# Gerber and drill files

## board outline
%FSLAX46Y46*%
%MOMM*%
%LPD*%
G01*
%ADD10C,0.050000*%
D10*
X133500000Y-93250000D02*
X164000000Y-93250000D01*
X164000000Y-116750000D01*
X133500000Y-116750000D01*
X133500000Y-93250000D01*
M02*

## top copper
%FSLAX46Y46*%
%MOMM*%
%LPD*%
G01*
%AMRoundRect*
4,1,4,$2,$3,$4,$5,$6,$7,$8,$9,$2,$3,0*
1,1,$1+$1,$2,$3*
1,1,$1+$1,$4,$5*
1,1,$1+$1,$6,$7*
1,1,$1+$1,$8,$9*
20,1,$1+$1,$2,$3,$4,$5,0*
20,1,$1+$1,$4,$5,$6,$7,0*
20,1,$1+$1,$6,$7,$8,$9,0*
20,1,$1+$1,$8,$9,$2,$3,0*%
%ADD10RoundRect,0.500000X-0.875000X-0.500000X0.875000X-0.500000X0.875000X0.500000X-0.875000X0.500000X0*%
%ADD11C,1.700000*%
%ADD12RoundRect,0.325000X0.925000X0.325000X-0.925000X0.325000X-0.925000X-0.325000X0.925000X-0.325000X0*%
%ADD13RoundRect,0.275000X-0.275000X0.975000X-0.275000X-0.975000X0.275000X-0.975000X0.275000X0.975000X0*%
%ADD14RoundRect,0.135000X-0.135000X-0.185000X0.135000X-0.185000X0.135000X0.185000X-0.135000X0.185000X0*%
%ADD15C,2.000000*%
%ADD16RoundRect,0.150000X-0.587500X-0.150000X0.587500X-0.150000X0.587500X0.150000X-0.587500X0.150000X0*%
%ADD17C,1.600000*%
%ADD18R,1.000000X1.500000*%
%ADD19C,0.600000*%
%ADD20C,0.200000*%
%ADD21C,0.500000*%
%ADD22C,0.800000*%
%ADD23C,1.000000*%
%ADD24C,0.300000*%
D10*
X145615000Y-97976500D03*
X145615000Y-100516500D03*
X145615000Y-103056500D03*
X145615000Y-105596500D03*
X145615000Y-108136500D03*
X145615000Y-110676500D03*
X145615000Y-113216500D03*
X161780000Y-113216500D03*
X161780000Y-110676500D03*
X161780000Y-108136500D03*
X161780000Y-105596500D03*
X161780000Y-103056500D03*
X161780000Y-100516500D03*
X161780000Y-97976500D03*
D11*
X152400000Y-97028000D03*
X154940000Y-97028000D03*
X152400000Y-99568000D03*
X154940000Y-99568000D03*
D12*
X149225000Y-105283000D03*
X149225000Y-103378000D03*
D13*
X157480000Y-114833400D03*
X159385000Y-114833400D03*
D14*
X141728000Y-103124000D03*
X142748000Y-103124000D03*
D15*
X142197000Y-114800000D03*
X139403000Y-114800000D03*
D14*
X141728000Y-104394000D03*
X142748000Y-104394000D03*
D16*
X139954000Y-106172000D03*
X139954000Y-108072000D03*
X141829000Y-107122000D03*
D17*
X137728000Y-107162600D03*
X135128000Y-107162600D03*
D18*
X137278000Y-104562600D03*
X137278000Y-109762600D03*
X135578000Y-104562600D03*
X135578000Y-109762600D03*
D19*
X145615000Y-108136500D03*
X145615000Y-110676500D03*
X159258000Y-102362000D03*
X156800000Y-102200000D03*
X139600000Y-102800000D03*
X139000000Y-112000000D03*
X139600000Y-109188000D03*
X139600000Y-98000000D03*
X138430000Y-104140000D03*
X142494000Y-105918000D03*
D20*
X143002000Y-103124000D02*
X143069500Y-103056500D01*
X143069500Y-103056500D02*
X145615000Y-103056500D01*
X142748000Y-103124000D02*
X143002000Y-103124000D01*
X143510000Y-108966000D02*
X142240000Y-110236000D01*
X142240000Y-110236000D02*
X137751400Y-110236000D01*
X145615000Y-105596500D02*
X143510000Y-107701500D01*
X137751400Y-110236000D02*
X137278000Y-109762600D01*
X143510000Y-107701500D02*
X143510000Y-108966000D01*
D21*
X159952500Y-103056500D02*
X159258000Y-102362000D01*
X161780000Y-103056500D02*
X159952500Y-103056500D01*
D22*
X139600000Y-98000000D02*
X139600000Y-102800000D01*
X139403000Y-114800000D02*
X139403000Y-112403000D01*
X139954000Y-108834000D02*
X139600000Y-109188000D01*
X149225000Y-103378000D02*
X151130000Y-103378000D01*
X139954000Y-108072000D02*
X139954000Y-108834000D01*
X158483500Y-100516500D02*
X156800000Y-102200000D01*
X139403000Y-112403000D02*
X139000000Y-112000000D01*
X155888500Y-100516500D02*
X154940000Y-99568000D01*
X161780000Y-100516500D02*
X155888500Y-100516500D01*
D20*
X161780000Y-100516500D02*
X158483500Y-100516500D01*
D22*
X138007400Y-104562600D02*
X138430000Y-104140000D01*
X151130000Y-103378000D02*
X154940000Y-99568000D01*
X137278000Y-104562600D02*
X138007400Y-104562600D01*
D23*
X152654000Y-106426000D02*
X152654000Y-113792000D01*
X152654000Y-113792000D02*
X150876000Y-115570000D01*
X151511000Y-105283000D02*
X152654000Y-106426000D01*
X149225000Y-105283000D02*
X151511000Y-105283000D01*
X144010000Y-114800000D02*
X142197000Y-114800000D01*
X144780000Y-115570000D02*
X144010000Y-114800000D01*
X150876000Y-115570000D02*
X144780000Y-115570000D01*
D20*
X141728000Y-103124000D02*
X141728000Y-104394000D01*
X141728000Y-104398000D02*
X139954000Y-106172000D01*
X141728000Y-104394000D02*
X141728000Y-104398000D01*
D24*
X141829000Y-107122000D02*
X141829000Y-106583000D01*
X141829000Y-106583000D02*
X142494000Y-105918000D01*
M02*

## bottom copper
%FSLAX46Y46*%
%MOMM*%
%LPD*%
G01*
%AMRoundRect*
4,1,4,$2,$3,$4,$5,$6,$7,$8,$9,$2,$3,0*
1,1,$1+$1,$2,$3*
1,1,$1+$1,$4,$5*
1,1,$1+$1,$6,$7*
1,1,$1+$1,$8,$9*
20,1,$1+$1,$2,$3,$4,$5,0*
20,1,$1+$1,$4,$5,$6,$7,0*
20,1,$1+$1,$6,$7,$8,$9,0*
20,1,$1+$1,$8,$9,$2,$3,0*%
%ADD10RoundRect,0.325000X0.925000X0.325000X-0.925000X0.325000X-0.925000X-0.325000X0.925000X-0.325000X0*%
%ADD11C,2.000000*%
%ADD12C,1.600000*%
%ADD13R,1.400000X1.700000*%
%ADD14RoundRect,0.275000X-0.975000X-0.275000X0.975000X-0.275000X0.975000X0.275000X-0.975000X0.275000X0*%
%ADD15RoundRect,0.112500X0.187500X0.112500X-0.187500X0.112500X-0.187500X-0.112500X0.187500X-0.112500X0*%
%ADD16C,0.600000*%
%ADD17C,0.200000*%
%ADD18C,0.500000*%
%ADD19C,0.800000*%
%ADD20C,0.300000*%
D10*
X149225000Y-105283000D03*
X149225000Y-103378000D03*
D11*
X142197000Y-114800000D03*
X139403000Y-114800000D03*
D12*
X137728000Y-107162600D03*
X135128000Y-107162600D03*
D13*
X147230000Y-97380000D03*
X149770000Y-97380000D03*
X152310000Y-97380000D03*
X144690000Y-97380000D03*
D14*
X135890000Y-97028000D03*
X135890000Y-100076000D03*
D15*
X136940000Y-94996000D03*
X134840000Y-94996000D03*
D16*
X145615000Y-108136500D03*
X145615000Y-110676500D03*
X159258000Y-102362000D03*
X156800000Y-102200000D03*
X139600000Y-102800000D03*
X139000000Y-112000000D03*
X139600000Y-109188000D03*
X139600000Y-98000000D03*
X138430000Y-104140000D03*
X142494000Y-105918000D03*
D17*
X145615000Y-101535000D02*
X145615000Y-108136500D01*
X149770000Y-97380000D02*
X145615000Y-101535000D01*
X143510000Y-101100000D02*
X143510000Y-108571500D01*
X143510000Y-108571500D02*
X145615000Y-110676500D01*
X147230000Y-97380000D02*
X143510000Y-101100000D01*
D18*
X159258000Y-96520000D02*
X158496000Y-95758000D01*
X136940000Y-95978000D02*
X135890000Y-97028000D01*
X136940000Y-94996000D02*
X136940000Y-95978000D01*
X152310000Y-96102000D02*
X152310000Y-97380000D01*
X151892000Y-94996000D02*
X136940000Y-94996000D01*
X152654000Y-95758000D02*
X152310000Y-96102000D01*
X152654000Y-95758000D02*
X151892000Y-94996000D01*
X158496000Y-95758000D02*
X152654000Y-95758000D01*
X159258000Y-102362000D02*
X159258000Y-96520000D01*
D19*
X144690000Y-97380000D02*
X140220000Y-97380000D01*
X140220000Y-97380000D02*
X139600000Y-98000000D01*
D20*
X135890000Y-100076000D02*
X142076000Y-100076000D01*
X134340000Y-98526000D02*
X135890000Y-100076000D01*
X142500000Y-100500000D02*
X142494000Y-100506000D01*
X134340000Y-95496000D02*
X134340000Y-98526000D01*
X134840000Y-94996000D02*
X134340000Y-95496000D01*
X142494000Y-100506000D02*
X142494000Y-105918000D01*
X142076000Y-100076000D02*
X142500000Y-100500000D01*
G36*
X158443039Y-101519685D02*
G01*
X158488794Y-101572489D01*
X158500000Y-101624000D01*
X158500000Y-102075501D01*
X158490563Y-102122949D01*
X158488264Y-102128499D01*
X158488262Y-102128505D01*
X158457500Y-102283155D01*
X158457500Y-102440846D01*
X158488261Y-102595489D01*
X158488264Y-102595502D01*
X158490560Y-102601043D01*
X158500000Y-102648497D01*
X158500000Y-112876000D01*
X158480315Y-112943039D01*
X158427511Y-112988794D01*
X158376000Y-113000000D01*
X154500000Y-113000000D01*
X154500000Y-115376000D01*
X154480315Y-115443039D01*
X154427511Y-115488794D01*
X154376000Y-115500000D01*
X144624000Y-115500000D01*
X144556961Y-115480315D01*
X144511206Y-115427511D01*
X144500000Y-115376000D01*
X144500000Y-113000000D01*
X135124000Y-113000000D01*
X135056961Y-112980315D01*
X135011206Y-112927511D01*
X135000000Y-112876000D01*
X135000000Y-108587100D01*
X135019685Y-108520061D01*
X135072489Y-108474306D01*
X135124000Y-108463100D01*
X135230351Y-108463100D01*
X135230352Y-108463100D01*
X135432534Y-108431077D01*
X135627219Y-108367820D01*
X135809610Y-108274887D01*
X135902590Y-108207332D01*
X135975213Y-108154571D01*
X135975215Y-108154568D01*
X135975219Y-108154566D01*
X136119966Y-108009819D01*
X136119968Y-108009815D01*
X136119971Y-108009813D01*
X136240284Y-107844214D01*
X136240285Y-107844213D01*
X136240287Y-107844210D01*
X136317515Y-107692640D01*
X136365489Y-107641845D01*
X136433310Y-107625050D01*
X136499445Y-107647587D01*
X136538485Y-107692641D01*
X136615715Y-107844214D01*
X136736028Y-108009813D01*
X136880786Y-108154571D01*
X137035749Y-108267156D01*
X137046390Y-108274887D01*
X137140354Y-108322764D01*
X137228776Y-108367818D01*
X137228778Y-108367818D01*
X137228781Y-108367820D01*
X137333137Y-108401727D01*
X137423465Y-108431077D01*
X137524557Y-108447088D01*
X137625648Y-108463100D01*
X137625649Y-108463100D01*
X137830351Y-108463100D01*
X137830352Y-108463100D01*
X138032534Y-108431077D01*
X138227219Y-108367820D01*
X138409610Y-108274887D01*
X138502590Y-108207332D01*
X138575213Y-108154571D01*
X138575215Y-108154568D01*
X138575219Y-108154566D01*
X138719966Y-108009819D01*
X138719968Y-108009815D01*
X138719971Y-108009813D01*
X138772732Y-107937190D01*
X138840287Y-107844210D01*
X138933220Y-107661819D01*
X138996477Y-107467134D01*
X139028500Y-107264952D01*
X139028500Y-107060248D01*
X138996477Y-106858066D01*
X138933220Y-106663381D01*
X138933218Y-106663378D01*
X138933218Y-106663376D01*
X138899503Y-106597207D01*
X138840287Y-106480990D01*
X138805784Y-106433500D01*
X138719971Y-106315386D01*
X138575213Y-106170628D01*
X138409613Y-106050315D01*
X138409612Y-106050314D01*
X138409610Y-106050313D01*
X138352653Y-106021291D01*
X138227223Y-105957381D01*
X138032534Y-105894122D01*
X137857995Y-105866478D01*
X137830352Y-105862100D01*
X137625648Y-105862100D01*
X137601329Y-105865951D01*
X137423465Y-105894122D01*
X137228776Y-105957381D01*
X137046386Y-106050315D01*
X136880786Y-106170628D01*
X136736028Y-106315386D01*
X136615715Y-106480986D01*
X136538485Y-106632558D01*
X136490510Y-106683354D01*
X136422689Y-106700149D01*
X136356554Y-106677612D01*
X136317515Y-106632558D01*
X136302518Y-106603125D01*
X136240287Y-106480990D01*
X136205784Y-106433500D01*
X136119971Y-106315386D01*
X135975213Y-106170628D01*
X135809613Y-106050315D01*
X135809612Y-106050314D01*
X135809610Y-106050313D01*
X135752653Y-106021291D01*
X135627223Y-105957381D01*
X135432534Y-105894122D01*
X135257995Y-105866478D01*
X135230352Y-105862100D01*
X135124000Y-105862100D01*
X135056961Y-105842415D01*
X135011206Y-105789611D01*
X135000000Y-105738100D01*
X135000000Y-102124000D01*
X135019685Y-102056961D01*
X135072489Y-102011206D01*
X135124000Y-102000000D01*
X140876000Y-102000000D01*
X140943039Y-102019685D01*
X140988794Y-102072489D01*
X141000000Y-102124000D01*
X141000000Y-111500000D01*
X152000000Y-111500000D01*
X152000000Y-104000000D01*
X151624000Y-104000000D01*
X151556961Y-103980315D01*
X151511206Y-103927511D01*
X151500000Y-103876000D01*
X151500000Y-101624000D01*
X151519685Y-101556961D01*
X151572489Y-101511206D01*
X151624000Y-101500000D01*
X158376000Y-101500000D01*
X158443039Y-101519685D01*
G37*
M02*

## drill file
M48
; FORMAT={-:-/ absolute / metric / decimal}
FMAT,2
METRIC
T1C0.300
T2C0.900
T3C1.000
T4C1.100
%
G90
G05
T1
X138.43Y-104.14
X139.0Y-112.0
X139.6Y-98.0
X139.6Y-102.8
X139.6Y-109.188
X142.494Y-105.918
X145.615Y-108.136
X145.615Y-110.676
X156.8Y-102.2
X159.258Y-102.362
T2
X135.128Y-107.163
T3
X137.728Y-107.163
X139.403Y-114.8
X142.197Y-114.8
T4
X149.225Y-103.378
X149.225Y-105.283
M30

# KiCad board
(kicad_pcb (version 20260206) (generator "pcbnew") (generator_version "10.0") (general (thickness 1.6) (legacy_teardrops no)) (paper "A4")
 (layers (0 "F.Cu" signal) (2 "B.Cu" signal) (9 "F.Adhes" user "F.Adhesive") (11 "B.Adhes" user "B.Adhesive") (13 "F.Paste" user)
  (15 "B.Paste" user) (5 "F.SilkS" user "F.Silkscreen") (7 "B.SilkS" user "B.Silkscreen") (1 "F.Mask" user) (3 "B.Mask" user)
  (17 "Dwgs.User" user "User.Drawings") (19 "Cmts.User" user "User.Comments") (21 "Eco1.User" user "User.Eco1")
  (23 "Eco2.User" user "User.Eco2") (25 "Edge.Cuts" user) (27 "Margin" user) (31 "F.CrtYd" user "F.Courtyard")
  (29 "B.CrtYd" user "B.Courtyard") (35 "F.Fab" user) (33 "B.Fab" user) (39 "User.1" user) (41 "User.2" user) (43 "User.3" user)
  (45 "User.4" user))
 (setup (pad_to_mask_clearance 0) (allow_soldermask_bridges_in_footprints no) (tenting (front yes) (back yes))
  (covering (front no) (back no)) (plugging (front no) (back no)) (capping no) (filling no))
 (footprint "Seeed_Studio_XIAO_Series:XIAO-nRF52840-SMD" (layer "F.Cu") (at 144.78 116.0965)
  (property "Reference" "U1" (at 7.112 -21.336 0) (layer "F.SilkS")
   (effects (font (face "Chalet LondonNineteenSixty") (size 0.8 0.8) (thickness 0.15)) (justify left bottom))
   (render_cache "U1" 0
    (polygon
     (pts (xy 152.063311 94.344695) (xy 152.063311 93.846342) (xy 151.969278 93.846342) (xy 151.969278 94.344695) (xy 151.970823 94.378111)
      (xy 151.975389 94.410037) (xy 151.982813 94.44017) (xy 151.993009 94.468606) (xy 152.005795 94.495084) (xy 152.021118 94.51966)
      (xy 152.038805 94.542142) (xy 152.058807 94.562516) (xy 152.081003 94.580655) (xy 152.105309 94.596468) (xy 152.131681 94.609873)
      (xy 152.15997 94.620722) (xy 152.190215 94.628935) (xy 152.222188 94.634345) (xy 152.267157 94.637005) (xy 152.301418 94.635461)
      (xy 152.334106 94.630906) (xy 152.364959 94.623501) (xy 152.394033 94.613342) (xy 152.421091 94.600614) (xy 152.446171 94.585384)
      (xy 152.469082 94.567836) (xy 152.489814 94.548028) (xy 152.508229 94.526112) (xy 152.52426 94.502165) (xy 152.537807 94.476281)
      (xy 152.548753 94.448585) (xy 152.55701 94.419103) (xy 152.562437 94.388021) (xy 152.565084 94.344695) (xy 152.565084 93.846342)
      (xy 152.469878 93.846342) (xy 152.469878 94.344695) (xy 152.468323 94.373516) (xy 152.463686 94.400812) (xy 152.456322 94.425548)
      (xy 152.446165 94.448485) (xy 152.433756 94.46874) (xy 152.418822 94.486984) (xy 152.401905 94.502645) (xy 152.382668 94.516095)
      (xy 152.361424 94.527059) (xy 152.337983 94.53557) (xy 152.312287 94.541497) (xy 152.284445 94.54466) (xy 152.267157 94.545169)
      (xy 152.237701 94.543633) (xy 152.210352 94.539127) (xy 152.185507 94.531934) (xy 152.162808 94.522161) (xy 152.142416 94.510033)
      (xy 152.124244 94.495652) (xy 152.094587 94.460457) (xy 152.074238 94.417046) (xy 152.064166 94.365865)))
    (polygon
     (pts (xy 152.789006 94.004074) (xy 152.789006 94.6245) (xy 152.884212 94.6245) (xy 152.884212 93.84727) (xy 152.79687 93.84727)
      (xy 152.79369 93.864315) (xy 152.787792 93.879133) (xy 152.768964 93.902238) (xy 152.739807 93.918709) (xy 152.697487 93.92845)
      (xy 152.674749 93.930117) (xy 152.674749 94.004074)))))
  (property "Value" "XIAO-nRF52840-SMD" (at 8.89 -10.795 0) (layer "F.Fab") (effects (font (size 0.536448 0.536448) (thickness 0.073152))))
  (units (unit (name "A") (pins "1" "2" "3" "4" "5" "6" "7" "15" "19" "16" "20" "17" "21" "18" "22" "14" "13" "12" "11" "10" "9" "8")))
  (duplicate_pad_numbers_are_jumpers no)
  (pad "1" smd roundrect (at 0.835 -18.12) (size 2.75 2) (layers "F.Cu" "F.Mask" "F.Paste") (roundrect_rratio 0.25)
   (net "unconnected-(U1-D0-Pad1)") (solder_mask_margin 0.0508) (thermal_bridge_angle 45))
  (pad "2" smd roundrect (at 0.835 -15.58) (size 2.75 2) (layers "F.Cu" "F.Mask" "F.Paste") (roundrect_rratio 0.25)
   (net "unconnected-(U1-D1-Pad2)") (solder_mask_margin 0.0508) (thermal_bridge_angle 45))
  (pad "3" smd roundrect (at 0.835 -13.04) (size 2.75 2) (layers "F.Cu" "F.Mask" "F.Paste") (roundrect_rratio 0.25) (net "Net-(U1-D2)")
   (solder_mask_margin 0.0508) (thermal_bridge_angle 45))
  (pad "4" smd roundrect (at 0.835 -10.5) (size 2.75 2) (layers "F.Cu" "F.Mask" "F.Paste") (roundrect_rratio 0.25) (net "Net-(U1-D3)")
   (solder_mask_margin 0.0508) (thermal_bridge_angle 45))
  (pad "5" smd roundrect (at 0.835 -7.96) (size 2.75 2) (layers "F.Cu" "F.Mask" "F.Paste") (roundrect_rratio 0.25) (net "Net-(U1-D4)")
   (solder_mask_margin 0.0508) (thermal_bridge_angle 45))
  (pad "6" smd roundrect (at 0.835 -5.42) (size 2.75 2) (layers "F.Cu" "F.Mask" "F.Paste") (roundrect_rratio 0.25) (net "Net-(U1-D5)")
   (solder_mask_margin 0.0508) (thermal_bridge_angle 45))
  (pad "7" smd roundrect (at 0.835 -2.88) (size 2.75 2) (layers "F.Cu" "F.Mask" "F.Paste") (roundrect_rratio 0.25)
   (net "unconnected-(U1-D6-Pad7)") (solder_mask_margin 0.0508) (thermal_bridge_angle 45))
  (pad "8" smd roundrect (at 17 -2.88) (size 2.75 2) (layers "F.Cu" "F.Mask" "F.Paste") (roundrect_rratio 0.25)
   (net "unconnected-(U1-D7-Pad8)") (solder_mask_margin 0.0508) (thermal_bridge_angle 45))
  (pad "9" smd roundrect (at 17 -5.42) (size 2.75 2) (layers "F.Cu" "F.Mask" "F.Paste") (roundrect_rratio 0.25)
   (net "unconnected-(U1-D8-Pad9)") (solder_mask_margin 0.0508) (thermal_bridge_angle 45))
  (pad "10" smd roundrect (at 17 -7.96) (size 2.75 2) (layers "F.Cu" "F.Mask" "F.Paste") (roundrect_rratio 0.25)
   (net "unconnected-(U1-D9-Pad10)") (solder_mask_margin 0.0508) (thermal_bridge_angle 45))
  (pad "11" smd roundrect (at 17 -10.5) (size 2.75 2) (layers "F.Cu" "F.Mask" "F.Paste") (roundrect_rratio 0.25)
   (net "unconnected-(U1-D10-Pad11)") (solder_mask_margin 0.0508) (thermal_bridge_angle 45))
  (pad "12" smd roundrect (at 17 -13.04) (size 2.75 2) (layers "F.Cu" "F.Mask" "F.Paste") (roundrect_rratio 0.25) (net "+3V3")
   (solder_mask_margin 0.0508) (thermal_bridge_angle 45))
  (pad "13" smd roundrect (at 17 -15.58) (size 2.75 2) (layers "F.Cu" "F.Mask" "F.Paste") (roundrect_rratio 0.25) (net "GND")
   (solder_mask_margin 0.0508) (thermal_bridge_angle 45))
  (pad "14" smd roundrect (at 17 -18.12) (size 2.75 2) (layers "F.Cu" "F.Mask" "F.Paste") (roundrect_rratio 0.25)
   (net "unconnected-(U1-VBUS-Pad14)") (solder_mask_margin 0.0508) (thermal_bridge_angle 45))
  (pad "15" smd circle (at 7.62 -19.0685) (size 1.7 1.7) (layers "F.Cu" "F.Mask" "F.Paste") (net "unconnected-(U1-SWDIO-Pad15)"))
  (pad "16" smd circle (at 10.16 -19.0685) (size 1.7 1.7) (layers "F.Cu" "F.Mask" "F.Paste") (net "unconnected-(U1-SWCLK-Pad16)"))
  (pad "17" smd circle (at 7.62 -16.5285) (size 1.7 1.7) (layers "F.Cu" "F.Mask" "F.Paste") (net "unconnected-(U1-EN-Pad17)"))
  (pad "18" smd circle (at 10.16 -16.5285) (size 1.7 1.7) (layers "F.Cu" "F.Mask" "F.Paste") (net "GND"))
  (pad "19" thru_hole roundrect (at 4.445 -10.8135 180) (size 2.5 1.3) (drill 1.1) (layers "*.Cu" "F.Mask" "F.Paste")
   (remove_unused_layers no) (roundrect_rratio 0.25) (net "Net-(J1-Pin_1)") (thermal_bridge_angle 45))
  (pad "20" thru_hole roundrect (at 4.445 -12.7185 180) (size 2.5 1.3) (drill 1.1) (layers "*.Cu" "F.Mask" "F.Paste")
   (remove_unused_layers no) (roundrect_rratio 0.25) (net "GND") (thermal_bridge_angle 45))
  (pad "21" smd roundrect (at 12.7 -1.2631 270) (size 2.5 1.1) (layers "F.Cu" "F.Mask" "F.Paste") (roundrect_rratio 0.25)
   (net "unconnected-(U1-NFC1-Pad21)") (thermal_bridge_angle 45))
  (pad "22" smd roundrect (at 14.605 -1.2631 270) (size 2.5 1.1) (layers "F.Cu" "F.Mask" "F.Paste") (roundrect_rratio 0.25)
   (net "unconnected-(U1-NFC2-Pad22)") (thermal_bridge_angle 45)))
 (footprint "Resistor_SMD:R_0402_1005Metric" (layer "F.Cu") (at 142.238 103.124)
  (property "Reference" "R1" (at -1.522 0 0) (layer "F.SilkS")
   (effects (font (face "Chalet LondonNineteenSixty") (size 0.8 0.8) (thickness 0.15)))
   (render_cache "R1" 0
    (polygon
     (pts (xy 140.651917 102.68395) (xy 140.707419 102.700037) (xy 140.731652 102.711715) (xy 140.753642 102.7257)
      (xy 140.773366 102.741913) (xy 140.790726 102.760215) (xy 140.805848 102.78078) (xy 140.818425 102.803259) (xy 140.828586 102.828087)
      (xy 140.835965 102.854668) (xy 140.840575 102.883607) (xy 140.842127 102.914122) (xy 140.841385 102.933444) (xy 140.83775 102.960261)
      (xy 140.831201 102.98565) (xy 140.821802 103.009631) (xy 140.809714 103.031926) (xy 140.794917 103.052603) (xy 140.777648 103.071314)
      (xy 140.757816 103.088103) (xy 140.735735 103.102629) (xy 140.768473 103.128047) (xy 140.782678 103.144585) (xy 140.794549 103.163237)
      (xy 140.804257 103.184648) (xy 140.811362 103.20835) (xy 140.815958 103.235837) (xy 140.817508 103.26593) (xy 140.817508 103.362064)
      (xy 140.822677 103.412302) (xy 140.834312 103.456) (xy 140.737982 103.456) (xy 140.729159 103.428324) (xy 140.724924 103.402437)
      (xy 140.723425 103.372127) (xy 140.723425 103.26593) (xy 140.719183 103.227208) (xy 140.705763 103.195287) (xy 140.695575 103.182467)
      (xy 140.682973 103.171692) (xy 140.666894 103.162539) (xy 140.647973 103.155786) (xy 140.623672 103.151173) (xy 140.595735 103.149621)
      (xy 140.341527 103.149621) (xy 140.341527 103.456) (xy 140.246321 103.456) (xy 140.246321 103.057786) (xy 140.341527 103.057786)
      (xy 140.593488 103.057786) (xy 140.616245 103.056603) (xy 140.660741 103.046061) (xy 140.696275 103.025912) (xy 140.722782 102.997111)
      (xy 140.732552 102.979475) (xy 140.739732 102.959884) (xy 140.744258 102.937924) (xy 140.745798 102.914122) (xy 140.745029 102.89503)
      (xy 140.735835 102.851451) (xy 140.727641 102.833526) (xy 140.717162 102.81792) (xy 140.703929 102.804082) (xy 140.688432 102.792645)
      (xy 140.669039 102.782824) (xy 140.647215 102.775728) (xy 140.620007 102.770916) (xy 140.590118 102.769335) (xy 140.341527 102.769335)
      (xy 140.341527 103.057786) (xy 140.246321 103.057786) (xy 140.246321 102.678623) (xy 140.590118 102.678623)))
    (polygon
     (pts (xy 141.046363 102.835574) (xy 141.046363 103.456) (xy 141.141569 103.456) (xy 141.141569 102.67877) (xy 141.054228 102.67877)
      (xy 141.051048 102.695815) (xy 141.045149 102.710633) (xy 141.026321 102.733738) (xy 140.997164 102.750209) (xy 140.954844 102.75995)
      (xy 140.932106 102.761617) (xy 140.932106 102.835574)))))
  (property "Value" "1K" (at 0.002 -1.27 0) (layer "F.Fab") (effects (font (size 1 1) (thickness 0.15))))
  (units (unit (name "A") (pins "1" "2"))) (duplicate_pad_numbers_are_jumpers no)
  (pad "1" smd roundrect (at -0.51 0) (size 0.54 0.64) (layers "F.Cu" "F.Mask" "F.Paste") (roundrect_rratio 0.25) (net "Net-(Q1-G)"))
  (pad "2" smd roundrect (at 0.51 0) (size 0.54 0.64) (layers "F.Cu" "F.Mask" "F.Paste") (roundrect_rratio 0.25) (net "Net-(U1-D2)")))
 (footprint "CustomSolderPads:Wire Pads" (layer "F.Cu") (at 140.8 114.8 -90)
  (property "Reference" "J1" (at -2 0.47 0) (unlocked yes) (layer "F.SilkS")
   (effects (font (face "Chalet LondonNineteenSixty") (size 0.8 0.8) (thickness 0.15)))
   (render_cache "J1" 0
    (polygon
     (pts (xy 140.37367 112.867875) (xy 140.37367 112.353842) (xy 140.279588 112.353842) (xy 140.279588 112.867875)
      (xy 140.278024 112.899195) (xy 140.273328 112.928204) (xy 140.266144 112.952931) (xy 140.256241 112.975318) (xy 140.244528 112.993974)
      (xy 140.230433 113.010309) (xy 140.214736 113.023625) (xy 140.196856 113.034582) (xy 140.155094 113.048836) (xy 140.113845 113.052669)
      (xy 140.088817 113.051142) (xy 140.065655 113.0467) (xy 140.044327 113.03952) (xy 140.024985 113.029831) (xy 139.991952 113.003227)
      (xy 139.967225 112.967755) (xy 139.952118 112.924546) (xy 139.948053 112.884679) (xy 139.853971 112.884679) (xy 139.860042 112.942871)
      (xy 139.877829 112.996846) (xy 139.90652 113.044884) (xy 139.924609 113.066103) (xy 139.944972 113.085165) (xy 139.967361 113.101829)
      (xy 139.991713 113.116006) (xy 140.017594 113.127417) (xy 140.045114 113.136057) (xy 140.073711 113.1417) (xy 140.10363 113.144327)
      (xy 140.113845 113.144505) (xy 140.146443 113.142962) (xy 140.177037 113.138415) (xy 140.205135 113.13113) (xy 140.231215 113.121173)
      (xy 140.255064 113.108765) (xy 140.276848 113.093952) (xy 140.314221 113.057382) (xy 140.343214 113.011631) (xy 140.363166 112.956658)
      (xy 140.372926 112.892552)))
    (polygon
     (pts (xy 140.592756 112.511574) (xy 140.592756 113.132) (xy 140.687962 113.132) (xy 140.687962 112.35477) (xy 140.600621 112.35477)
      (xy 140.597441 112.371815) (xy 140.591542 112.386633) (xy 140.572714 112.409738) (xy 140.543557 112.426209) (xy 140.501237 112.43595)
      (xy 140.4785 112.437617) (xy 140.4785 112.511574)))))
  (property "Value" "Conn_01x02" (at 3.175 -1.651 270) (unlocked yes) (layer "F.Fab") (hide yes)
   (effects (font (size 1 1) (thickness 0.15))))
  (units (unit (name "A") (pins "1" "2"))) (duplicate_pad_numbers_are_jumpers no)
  (pad "1" thru_hole circle (at 0 -1.397 90) (size 2 2) (drill 1) (layers "*.Cu" "*.Mask") (remove_unused_layers no) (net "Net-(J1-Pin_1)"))
  (pad "2" thru_hole circle (at 0 1.397 90) (size 2 2) (drill 1) (layers "*.Cu" "*.Mask") (remove_unused_layers no) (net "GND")))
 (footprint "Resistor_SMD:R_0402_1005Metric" (layer "F.Cu") (at 142.238 104.394)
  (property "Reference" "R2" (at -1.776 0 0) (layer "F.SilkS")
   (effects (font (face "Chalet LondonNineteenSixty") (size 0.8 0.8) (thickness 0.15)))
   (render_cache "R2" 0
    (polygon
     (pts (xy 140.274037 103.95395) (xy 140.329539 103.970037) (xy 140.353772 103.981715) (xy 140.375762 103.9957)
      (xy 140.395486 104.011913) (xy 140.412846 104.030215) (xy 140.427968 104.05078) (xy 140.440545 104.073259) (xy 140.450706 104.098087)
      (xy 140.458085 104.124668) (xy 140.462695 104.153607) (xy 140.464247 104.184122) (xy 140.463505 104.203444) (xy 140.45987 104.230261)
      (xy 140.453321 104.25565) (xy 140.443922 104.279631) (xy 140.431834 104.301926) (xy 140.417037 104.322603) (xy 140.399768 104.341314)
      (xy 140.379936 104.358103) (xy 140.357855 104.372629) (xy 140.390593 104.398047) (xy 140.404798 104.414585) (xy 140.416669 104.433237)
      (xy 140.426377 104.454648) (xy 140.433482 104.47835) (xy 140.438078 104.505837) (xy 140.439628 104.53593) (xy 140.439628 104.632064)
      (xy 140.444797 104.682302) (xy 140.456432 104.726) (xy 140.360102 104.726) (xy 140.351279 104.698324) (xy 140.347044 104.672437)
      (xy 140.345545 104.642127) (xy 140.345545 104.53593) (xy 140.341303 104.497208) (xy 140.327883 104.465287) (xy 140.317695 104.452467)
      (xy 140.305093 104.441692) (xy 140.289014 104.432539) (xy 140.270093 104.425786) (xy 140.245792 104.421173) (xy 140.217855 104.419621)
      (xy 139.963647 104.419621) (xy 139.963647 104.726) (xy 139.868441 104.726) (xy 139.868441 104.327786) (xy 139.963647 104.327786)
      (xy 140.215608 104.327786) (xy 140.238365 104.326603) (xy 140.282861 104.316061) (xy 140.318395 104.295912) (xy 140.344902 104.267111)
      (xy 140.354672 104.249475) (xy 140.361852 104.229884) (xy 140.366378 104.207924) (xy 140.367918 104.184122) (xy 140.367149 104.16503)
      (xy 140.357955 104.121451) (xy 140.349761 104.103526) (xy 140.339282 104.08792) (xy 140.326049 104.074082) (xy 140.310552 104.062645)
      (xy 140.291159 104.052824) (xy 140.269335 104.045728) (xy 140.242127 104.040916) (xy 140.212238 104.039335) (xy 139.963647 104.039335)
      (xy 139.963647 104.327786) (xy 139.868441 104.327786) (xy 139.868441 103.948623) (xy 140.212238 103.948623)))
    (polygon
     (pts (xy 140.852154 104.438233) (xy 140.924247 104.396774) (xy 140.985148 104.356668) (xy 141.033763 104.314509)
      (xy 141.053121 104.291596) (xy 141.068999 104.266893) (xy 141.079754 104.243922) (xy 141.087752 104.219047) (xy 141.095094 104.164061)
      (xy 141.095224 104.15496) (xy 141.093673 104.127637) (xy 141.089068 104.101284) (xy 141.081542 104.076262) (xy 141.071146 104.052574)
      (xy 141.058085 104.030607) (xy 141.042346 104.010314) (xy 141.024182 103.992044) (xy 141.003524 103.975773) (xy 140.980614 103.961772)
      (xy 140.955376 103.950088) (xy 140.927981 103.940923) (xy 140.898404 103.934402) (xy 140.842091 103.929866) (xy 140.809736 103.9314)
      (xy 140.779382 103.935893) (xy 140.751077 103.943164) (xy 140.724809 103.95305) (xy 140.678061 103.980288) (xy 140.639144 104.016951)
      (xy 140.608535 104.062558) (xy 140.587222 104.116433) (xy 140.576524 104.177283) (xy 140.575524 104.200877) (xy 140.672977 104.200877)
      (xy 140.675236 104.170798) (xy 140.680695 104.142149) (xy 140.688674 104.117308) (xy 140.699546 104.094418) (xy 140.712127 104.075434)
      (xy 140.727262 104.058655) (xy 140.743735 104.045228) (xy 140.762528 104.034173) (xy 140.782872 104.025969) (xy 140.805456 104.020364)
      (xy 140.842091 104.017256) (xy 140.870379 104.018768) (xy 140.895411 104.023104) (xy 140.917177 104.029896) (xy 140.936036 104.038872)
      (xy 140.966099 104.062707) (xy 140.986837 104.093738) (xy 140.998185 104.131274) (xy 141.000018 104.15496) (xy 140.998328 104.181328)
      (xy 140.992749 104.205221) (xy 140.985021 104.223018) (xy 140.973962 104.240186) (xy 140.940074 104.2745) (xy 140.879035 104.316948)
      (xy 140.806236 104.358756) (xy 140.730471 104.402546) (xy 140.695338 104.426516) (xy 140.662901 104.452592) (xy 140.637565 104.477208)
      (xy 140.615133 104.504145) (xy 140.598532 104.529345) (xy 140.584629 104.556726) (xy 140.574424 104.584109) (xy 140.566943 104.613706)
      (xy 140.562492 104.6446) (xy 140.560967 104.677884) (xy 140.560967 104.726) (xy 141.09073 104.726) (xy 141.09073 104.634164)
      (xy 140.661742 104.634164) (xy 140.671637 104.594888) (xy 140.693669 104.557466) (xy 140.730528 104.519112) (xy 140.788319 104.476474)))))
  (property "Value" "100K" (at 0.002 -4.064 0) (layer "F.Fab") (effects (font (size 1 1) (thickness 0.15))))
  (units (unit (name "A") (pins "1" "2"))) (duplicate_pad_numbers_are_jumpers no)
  (pad "1" smd roundrect (at -0.51 0) (size 0.54 0.64) (layers "F.Cu" "F.Mask" "F.Paste") (roundrect_rratio 0.25) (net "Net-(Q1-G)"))
  (pad "2" smd roundrect (at 0.51 0) (size 0.54 0.64) (layers "F.Cu" "F.Mask" "F.Paste") (roundrect_rratio 0.25) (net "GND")))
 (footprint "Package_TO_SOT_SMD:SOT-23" (layer "F.Cu") (at 140.8915 107.122)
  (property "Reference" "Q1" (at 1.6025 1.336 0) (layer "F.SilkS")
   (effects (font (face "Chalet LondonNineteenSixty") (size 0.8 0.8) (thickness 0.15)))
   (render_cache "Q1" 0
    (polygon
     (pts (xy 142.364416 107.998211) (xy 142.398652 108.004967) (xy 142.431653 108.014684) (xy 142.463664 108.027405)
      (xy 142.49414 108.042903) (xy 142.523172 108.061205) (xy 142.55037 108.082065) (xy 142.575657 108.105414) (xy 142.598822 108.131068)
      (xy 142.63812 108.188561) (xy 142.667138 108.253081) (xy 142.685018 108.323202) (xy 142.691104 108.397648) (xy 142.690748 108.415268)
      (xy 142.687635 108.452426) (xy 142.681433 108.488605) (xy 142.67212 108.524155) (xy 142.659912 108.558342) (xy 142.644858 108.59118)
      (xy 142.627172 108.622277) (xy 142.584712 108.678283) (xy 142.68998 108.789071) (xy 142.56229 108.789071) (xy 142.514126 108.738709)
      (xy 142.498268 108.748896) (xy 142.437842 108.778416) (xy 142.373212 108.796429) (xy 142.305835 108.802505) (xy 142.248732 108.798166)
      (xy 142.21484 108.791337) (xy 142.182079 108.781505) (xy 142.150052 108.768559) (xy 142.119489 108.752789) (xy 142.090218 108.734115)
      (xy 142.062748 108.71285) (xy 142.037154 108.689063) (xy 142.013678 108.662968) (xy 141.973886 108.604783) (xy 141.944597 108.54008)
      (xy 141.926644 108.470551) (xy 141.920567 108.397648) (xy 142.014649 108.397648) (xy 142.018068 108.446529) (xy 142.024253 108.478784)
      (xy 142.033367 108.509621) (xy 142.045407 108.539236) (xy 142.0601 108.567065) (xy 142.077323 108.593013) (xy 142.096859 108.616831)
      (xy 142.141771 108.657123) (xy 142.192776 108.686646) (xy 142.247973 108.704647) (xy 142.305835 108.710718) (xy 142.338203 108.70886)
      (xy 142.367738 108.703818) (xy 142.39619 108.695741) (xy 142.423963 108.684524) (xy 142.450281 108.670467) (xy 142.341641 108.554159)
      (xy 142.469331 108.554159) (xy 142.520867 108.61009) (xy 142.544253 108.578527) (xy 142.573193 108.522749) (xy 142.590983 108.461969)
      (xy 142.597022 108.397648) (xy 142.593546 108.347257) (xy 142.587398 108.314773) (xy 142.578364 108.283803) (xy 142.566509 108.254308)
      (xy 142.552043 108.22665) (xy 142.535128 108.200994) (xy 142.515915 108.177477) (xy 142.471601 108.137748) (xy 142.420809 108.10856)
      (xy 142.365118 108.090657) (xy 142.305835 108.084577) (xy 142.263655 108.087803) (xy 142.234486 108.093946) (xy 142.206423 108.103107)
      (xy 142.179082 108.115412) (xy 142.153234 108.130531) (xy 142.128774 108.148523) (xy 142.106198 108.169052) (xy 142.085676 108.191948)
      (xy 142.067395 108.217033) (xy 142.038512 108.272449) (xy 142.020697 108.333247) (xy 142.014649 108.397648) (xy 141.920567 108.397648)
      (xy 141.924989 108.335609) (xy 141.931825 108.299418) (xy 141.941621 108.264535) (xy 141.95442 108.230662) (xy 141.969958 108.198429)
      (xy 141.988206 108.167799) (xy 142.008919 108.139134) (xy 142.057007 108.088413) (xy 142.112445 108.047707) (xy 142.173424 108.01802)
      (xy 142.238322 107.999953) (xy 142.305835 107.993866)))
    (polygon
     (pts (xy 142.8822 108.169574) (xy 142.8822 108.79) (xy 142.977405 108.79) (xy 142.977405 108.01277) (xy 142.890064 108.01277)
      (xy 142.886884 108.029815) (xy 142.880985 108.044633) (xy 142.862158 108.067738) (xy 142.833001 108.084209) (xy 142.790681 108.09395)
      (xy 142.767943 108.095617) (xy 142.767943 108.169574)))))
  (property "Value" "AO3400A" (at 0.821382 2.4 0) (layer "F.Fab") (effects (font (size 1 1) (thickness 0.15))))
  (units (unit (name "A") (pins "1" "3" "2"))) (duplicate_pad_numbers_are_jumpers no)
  (pad "1" smd roundrect (at -0.9375 -0.95) (size 1.475 0.6) (layers "F.Cu" "F.Mask" "F.Paste") (roundrect_rratio 0.25) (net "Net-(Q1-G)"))
  (pad "2" smd roundrect (at -0.9375 0.95) (size 1.475 0.6) (layers "F.Cu" "F.Mask" "F.Paste") (roundrect_rratio 0.25) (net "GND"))
  (pad "3" smd roundrect (at 0.9375 0) (size 1.475 0.6) (layers "F.Cu" "F.Mask" "F.Paste") (roundrect_rratio 0.25) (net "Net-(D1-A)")))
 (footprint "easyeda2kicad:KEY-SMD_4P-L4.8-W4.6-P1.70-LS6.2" (layer "F.Cu") (at 136.428 107.1626 -90)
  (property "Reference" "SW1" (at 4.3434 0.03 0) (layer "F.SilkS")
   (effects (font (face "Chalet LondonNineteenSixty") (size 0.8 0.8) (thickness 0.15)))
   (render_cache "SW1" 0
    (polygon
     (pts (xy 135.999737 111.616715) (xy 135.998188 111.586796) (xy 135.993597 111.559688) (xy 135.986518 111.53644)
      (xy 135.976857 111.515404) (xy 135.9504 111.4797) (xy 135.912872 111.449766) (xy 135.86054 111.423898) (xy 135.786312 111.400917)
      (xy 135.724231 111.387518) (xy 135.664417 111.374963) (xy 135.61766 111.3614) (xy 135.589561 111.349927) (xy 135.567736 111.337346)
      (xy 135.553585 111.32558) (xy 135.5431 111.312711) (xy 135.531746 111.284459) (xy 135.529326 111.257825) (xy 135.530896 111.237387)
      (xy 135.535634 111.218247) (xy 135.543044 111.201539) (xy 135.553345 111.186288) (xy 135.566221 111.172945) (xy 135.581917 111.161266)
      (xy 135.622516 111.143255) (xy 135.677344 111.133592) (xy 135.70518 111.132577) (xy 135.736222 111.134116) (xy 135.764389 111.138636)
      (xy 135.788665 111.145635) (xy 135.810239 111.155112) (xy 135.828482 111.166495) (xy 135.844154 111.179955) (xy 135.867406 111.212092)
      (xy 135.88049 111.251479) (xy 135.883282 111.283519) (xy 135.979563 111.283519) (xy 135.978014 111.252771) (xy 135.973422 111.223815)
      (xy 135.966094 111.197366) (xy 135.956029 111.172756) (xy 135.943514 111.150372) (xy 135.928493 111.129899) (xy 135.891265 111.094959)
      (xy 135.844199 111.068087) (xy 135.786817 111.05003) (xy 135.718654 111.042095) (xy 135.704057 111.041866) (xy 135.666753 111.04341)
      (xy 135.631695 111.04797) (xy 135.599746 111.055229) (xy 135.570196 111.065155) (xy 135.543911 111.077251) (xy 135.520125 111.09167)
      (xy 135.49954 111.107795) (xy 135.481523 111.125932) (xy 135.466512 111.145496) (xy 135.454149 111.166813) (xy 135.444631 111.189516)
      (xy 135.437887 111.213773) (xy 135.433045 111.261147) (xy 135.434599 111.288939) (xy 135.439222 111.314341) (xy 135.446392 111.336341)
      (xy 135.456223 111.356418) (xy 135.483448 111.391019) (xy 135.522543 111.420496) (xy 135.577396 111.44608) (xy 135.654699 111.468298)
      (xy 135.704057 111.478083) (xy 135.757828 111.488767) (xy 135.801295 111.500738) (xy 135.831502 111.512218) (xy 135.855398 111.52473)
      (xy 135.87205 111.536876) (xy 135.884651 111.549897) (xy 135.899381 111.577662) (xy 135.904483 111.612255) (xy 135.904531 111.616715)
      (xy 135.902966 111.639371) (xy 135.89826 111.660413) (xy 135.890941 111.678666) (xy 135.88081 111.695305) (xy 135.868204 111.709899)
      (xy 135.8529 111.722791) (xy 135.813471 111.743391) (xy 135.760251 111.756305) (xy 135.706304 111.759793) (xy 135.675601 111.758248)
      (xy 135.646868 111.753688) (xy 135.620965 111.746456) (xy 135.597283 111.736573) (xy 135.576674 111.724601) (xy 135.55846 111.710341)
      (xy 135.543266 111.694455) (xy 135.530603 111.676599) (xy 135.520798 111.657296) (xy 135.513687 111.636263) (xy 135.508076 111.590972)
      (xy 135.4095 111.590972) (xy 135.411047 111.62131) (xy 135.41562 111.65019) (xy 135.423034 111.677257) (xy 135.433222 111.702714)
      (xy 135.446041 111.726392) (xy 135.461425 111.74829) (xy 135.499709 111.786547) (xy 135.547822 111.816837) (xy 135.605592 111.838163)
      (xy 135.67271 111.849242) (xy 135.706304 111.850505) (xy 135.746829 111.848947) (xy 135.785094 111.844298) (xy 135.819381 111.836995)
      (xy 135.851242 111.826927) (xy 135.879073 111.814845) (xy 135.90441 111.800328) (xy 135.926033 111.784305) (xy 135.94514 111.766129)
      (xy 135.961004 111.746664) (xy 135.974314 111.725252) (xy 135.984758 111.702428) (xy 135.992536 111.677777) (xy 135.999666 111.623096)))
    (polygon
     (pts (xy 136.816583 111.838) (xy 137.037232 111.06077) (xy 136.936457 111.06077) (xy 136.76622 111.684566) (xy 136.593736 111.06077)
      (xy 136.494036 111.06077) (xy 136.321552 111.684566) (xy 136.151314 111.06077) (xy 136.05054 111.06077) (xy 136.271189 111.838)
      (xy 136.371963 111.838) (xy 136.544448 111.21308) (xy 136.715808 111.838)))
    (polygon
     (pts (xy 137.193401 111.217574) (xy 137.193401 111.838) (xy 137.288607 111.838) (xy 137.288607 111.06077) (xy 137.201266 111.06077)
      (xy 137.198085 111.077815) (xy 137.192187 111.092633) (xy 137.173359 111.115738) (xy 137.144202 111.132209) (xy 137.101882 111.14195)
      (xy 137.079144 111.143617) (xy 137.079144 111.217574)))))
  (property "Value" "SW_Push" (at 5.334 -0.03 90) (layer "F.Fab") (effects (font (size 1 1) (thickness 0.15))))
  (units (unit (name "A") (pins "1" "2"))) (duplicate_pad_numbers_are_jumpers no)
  (pad "" thru_hole circle (at 0 -1.3 270) (size 1.6 1.6) (drill 1) (layers "*.Cu" "*.Mask") (remove_unused_layers no))
  (pad "" thru_hole circle (at 0 1.3 270) (size 1.6 1.6) (drill 0.9) (layers "*.Cu" "*.Mask") (remove_unused_layers no))
  (pad "1" smd rect (at -2.6 -0.85 270) (size 1.5 1) (layers "F.Cu" "F.Mask" "F.Paste") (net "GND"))
  (pad "2" smd rect (at 2.6 -0.85 270) (size 1.5 1) (layers "F.Cu" "F.Mask" "F.Paste") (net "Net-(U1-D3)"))
  (pad "3" smd rect (at -2.6 0.85 270) (size 1.5 1) (layers "F.Cu" "F.Mask" "F.Paste"))
  (pad "4" smd rect (at 2.6 0.85 270) (size 1.5 1) (layers "F.Cu" "F.Mask" "F.Paste")))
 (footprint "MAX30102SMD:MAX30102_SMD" (layer "B.Cu") (at 148.5 105 180)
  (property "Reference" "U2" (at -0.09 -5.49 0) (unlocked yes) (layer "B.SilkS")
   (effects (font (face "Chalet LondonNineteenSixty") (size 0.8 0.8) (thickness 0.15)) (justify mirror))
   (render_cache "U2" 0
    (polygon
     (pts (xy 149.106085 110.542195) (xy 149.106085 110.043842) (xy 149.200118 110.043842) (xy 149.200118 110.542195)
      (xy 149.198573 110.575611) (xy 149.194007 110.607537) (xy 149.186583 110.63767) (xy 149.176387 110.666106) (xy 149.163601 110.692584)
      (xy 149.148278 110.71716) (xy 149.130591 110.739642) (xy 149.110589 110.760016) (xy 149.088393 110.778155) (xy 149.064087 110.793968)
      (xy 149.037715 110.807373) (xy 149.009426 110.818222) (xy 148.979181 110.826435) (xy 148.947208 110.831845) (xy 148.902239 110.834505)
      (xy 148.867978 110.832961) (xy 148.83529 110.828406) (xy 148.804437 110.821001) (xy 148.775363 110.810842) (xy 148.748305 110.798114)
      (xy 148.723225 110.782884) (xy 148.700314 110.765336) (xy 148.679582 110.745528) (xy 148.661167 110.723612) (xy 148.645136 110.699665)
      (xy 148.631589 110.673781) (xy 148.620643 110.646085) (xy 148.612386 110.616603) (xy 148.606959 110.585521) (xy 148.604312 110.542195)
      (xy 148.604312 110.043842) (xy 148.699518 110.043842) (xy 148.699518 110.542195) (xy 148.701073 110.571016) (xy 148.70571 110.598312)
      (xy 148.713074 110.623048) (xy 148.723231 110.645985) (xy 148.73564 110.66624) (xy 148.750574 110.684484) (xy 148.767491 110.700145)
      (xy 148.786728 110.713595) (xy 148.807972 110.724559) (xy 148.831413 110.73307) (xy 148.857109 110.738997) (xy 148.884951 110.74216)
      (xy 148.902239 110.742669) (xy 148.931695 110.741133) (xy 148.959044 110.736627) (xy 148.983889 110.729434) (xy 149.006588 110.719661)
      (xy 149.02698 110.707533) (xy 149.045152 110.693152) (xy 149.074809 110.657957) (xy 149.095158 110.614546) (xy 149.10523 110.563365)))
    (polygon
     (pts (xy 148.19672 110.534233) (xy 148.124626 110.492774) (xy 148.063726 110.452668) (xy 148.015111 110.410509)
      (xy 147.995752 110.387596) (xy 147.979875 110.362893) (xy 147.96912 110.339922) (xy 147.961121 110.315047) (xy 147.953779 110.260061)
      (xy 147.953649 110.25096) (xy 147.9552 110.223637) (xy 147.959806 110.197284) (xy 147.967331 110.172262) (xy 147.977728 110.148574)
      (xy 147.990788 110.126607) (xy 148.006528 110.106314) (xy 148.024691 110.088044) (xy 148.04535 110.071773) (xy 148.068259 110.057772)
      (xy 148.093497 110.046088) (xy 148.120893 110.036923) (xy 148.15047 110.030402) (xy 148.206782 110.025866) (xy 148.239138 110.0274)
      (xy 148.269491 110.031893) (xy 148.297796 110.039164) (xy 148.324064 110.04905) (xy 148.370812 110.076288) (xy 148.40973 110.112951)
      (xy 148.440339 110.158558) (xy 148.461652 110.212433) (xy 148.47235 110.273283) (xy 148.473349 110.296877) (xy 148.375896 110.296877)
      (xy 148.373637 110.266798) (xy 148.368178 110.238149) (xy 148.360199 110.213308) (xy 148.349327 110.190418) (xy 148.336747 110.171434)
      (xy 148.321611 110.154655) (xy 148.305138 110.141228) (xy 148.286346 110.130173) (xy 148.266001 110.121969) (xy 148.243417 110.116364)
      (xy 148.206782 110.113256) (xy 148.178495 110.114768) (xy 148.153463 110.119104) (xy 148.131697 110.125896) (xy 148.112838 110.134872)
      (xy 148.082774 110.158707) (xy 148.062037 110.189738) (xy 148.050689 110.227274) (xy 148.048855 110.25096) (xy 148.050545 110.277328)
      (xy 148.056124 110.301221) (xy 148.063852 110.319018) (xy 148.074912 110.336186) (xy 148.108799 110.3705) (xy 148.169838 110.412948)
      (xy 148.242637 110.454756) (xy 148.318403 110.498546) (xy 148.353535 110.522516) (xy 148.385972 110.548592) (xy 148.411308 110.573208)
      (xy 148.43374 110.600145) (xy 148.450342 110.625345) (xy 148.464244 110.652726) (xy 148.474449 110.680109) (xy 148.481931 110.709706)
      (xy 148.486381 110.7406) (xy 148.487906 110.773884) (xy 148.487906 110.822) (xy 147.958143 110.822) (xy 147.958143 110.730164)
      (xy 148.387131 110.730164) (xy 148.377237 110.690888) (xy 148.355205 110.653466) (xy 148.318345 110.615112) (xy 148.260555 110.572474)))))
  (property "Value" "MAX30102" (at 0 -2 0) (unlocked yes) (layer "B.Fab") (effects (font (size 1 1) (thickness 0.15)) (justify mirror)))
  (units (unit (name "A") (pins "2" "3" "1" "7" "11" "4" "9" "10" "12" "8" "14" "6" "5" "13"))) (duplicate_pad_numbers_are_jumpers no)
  (pad "2" smd rect (at 1.27 7.62 180) (size 1.4 1.7) (layers "B.Cu" "B.Mask") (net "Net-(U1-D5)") (thermal_bridge_angle 45))
  (pad "3" smd rect (at -1.27 7.62 180) (size 1.4 1.7) (layers "B.Cu" "B.Mask") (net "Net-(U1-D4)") (thermal_bridge_angle 45))
  (pad "11" smd rect (at -3.81 7.62 180) (size 1.4 1.7) (layers "B.Cu" "B.Mask") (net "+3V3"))
  (pad "12" smd rect (at 3.81 7.62 180) (size 1.4 1.7) (layers "B.Cu" "B.Mask") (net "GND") (thermal_bridge_angle 45))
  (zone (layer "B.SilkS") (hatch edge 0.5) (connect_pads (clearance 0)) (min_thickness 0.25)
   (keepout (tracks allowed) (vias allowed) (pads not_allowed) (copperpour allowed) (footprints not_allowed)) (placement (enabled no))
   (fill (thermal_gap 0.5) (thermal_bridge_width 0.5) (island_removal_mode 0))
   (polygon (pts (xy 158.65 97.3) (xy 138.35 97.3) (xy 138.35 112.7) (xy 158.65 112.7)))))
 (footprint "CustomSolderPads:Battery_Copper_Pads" (layer "B.Cu") (at 135.89 98.552 180)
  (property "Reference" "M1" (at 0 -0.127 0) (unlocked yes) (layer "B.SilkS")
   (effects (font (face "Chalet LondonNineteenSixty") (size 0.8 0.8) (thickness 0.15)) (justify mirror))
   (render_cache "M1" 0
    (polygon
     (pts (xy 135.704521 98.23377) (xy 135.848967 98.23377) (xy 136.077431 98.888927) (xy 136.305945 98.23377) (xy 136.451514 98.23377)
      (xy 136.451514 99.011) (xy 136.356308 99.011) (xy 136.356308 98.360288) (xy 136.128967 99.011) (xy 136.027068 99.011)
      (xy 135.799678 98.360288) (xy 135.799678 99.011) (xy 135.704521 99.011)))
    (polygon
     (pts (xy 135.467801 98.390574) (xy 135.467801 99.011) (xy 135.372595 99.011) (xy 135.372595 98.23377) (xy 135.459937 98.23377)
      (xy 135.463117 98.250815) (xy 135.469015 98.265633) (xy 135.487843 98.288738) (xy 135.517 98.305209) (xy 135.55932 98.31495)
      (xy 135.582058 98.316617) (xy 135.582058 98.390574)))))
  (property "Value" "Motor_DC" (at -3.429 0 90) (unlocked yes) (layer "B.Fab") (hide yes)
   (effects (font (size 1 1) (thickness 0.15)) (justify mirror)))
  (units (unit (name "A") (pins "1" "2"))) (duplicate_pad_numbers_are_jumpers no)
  (pad "1" smd roundrect (at 0 1.524) (size 2.5 1.1) (layers "B.Cu" "B.Mask" "B.Paste") (roundrect_rratio 0.25) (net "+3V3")
   (thermal_bridge_angle 45))
  (pad "2" smd roundrect (at 0 -1.524) (size 2.5 1.1) (layers "B.Cu" "B.Mask" "B.Paste") (roundrect_rratio 0.25) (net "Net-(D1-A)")
   (thermal_bridge_angle 45)))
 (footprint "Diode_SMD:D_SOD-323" (layer "B.Cu") (at 135.89 94.996 180)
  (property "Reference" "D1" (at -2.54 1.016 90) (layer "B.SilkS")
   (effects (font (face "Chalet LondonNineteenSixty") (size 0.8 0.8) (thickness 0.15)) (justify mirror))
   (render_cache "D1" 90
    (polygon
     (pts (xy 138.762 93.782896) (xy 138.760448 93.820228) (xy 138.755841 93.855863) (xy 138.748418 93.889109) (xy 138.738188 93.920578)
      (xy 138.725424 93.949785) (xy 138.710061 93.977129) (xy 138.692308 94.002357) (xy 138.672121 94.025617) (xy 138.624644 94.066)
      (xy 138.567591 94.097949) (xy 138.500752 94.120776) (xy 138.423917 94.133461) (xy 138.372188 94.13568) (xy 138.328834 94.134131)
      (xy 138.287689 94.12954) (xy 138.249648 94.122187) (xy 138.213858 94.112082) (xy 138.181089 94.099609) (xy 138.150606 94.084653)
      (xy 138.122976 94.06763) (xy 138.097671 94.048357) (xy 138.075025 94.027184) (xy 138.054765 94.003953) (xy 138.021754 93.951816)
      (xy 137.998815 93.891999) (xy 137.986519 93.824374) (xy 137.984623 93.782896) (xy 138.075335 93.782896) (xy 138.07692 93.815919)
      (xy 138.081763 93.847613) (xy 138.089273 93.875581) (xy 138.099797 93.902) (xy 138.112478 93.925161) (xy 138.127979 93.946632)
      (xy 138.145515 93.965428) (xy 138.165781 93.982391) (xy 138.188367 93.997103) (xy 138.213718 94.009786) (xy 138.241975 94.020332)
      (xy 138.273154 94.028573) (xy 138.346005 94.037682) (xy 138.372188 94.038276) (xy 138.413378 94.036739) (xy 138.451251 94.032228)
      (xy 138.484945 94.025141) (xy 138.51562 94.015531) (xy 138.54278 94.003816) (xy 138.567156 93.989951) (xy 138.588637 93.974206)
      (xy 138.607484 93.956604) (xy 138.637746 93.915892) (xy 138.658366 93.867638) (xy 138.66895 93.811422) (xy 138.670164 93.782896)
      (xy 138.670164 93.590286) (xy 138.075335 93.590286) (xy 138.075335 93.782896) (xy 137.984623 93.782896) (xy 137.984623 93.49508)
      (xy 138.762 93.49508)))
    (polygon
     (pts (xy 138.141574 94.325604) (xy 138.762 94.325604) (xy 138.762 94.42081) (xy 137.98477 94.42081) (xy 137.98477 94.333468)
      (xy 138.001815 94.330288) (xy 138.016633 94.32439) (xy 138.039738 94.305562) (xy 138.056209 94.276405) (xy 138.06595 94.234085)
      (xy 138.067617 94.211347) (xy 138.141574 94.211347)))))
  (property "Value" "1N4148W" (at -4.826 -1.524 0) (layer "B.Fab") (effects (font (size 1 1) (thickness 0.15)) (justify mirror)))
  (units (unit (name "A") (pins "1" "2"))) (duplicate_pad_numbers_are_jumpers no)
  (pad "1" smd roundrect (at -1.05 0 180) (size 0.6 0.45) (layers "B.Cu" "B.Mask" "B.Paste") (roundrect_rratio 0.25) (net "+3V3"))
  (pad "2" smd roundrect (at 1.05 0 180) (size 0.6 0.45) (layers "B.Cu" "B.Mask" "B.Paste") (roundrect_rratio 0.25) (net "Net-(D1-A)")))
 (gr_rect (start 133.5 93.25) (end 164 116.75) (stroke (width 0.05) (type default)) (fill no) (layer "Edge.Cuts"))
 (segment (start 143.002 103.124) (end 143.0695 103.0565) (width 0.2) (layer "F.Cu") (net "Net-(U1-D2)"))
 (segment (start 143.0695 103.0565) (end 145.615 103.0565) (width 0.2) (layer "F.Cu") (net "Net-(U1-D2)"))
 (segment (start 142.748 103.124) (end 143.002 103.124) (width 0.2) (layer "F.Cu") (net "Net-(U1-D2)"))
 (segment (start 143.51 108.966) (end 142.24 110.236) (width 0.2) (layer "F.Cu") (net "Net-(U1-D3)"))
 (segment (start 142.24 110.236) (end 137.7514 110.236) (width 0.2) (layer "F.Cu") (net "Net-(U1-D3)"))
 (segment (start 145.615 105.5965) (end 143.51 107.7015) (width 0.2) (layer "F.Cu") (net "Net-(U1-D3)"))
 (segment (start 137.7514 110.236) (end 137.278 109.7626) (width 0.2) (layer "F.Cu") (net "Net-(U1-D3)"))
 (segment (start 143.51 107.7015) (end 143.51 108.966) (width 0.2) (layer "F.Cu") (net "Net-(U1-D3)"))
 (via (at 145.615 108.1365) (size 0.6) (drill 0.3) (layers "F.Cu" "B.Cu") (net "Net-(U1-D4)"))
 (segment (start 145.615 101.535) (end 145.615 108.1365) (width 0.2) (layer "B.Cu") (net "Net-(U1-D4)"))
 (segment (start 149.77 97.38) (end 145.615 101.535) (width 0.2) (layer "B.Cu") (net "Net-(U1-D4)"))
 (via (at 145.615 110.6765) (size 0.6) (drill 0.3) (layers "F.Cu" "B.Cu") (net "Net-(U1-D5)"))
 (segment (start 143.51 101.1) (end 143.51 108.5715) (width 0.2) (layer "B.Cu") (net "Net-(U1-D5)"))
 (segment (start 143.51 108.5715) (end 145.615 110.6765) (width 0.2) (layer "B.Cu") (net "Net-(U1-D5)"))
 (segment (start 147.23 97.38) (end 143.51 101.1) (width 0.2) (layer "B.Cu") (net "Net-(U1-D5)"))
 (segment (start 159.9525 103.0565) (end 159.258 102.362) (width 0.5) (layer "F.Cu") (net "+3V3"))
 (segment (start 161.78 103.0565) (end 159.9525 103.0565) (width 0.5) (layer "F.Cu") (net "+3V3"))
 (via (at 159.258 102.362) (size 0.6) (drill 0.3) (layers "F.Cu" "B.Cu") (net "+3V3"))
 (segment (start 159.258 96.52) (end 158.496 95.758) (width 0.5) (layer "B.Cu") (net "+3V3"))
 (segment (start 136.94 95.978) (end 135.89 97.028) (width 0.5) (layer "B.Cu") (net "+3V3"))
 (segment (start 136.94 94.996) (end 136.94 95.978) (width 0.5) (layer "B.Cu") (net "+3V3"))
 (segment (start 152.31 96.102) (end 152.31 97.38) (width 0.5) (layer "B.Cu") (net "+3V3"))
 (segment (start 151.892 94.996) (end 136.94 94.996) (width 0.5) (layer "B.Cu") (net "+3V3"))
 (segment (start 152.654 95.758) (end 152.31 96.102) (width 0.5) (layer "B.Cu") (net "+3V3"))
 (segment (start 152.654 95.758) (end 151.892 94.996) (width 0.5) (layer "B.Cu") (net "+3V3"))
 (segment (start 158.496 95.758) (end 152.654 95.758) (width 0.5) (layer "B.Cu") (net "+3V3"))
 (segment (start 159.258 102.362) (end 159.258 96.52) (width 0.5) (layer "B.Cu") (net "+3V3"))
 (segment (start 139.6 98) (end 139.6 102.8) (width 0.8) (layer "F.Cu") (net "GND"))
 (segment (start 139.403 114.8) (end 139.403 112.403) (width 0.8) (layer "F.Cu") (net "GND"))
 (segment (start 139.954 108.834) (end 139.6 109.188) (width 0.8) (layer "F.Cu") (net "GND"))
 (segment (start 149.225 103.378) (end 151.13 103.378) (width 0.8) (layer "F.Cu") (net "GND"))
 (segment (start 139.954 108.072) (end 139.954 108.834) (width 0.8) (layer "F.Cu") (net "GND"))
 (segment (start 158.4835 100.5165) (end 156.8 102.2) (width 0.8) (layer "F.Cu") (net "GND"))
 (segment (start 139.403 112.403) (end 139 112) (width 0.8) (layer "F.Cu") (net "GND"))
 (segment (start 155.8885 100.5165) (end 154.94 99.568) (width 0.8) (layer "F.Cu") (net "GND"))
 (segment (start 161.78 100.5165) (end 155.8885 100.5165) (width 0.8) (layer "F.Cu") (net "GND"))
 (segment (start 161.78 100.5165) (end 158.4835 100.5165) (width 0.2) (layer "F.Cu") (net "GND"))
 (segment (start 138.0074 104.5626) (end 138.43 104.14) (width 0.8) (layer "F.Cu") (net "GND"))
 (segment (start 151.13 103.378) (end 154.94 99.568) (width 0.8) (layer "F.Cu") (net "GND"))
 (segment (start 137.278 104.5626) (end 138.0074 104.5626) (width 0.8) (layer "F.Cu") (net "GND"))
 (via (at 156.8 102.2) (size 0.6) (drill 0.3) (layers "F.Cu" "B.Cu") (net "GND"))
 (via (at 139.6 102.8) (size 0.6) (drill 0.3) (layers "F.Cu" "B.Cu") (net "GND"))
 (via (at 139 112) (size 0.6) (drill 0.3) (layers "F.Cu" "B.Cu") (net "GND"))
 (via (at 139.6 109.188) (size 0.6) (drill 0.3) (layers "F.Cu" "B.Cu") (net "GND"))
 (via (at 139.6 98) (size 0.6) (drill 0.3) (layers "F.Cu" "B.Cu") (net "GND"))
 (via (at 138.43 104.14) (size 0.6) (drill 0.3) (layers "F.Cu" "B.Cu") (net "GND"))
 (segment (start 144.69 97.38) (end 140.22 97.38) (width 0.8) (layer "B.Cu") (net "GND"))
 (segment (start 140.22 97.38) (end 139.6 98) (width 0.8) (layer "B.Cu") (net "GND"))
 (segment (start 152.654 106.426) (end 152.654 113.792) (width 1) (layer "F.Cu") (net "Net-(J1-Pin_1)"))
 (segment (start 152.654 113.792) (end 150.876 115.57) (width 1) (layer "F.Cu") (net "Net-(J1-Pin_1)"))
 (segment (start 151.511 105.283) (end 152.654 106.426) (width 1) (layer "F.Cu") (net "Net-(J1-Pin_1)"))
 (segment (start 149.225 105.283) (end 151.511 105.283) (width 1) (layer "F.Cu") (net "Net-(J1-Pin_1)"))
 (segment (start 144.01 114.8) (end 142.197 114.8) (width 1) (layer "F.Cu") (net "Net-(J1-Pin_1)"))
 (segment (start 144.78 115.57) (end 144.01 114.8) (width 1) (layer "F.Cu") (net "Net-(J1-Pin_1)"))
 (segment (start 150.876 115.57) (end 144.78 115.57) (width 1) (layer "F.Cu") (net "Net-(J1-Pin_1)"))
 (segment (start 141.728 103.124) (end 141.728 104.394) (width 0.2) (layer "F.Cu") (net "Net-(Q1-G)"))
 (segment (start 141.728 104.398) (end 139.954 106.172) (width 0.2) (layer "F.Cu") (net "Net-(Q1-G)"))
 (segment (start 141.728 104.394) (end 141.728 104.398) (width 0.2) (layer "F.Cu") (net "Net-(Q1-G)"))
 (segment (start 141.829 107.122) (end 141.829 106.583) (width 0.3) (layer "F.Cu") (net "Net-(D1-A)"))
 (segment (start 141.829 106.583) (end 142.494 105.918) (width 0.3) (layer "F.Cu") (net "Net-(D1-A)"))
 (via (at 142.494 105.918) (size 0.6) (drill 0.3) (layers "F.Cu" "B.Cu") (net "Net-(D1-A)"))
 (segment (start 135.89 100.076) (end 142.076 100.076) (width 0.3) (layer "B.Cu") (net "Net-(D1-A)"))
 (segment (start 134.34 98.526) (end 135.89 100.076) (width 0.3) (layer "B.Cu") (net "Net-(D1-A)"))
 (segment (start 142.5 100.5) (end 142.494 100.506) (width 0.3) (layer "B.Cu") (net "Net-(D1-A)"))
 (segment (start 134.34 95.496) (end 134.34 98.526) (width 0.3) (layer "B.Cu") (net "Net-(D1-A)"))
 (segment (start 134.84 94.996) (end 134.34 95.496) (width 0.3) (layer "B.Cu") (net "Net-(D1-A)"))
 (segment (start 142.494 100.506) (end 142.494 105.918) (width 0.3) (layer "B.Cu") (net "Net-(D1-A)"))
 (segment (start 142.076 100.076) (end 142.5 100.5) (width 0.3) (layer "B.Cu") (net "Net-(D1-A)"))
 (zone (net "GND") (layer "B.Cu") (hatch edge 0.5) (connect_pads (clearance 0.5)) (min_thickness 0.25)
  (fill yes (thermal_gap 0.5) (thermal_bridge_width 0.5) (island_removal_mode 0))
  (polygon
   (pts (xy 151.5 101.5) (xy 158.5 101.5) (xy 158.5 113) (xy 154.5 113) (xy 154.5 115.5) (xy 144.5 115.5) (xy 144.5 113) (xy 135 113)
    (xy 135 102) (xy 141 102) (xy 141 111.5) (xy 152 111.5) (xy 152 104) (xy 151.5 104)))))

